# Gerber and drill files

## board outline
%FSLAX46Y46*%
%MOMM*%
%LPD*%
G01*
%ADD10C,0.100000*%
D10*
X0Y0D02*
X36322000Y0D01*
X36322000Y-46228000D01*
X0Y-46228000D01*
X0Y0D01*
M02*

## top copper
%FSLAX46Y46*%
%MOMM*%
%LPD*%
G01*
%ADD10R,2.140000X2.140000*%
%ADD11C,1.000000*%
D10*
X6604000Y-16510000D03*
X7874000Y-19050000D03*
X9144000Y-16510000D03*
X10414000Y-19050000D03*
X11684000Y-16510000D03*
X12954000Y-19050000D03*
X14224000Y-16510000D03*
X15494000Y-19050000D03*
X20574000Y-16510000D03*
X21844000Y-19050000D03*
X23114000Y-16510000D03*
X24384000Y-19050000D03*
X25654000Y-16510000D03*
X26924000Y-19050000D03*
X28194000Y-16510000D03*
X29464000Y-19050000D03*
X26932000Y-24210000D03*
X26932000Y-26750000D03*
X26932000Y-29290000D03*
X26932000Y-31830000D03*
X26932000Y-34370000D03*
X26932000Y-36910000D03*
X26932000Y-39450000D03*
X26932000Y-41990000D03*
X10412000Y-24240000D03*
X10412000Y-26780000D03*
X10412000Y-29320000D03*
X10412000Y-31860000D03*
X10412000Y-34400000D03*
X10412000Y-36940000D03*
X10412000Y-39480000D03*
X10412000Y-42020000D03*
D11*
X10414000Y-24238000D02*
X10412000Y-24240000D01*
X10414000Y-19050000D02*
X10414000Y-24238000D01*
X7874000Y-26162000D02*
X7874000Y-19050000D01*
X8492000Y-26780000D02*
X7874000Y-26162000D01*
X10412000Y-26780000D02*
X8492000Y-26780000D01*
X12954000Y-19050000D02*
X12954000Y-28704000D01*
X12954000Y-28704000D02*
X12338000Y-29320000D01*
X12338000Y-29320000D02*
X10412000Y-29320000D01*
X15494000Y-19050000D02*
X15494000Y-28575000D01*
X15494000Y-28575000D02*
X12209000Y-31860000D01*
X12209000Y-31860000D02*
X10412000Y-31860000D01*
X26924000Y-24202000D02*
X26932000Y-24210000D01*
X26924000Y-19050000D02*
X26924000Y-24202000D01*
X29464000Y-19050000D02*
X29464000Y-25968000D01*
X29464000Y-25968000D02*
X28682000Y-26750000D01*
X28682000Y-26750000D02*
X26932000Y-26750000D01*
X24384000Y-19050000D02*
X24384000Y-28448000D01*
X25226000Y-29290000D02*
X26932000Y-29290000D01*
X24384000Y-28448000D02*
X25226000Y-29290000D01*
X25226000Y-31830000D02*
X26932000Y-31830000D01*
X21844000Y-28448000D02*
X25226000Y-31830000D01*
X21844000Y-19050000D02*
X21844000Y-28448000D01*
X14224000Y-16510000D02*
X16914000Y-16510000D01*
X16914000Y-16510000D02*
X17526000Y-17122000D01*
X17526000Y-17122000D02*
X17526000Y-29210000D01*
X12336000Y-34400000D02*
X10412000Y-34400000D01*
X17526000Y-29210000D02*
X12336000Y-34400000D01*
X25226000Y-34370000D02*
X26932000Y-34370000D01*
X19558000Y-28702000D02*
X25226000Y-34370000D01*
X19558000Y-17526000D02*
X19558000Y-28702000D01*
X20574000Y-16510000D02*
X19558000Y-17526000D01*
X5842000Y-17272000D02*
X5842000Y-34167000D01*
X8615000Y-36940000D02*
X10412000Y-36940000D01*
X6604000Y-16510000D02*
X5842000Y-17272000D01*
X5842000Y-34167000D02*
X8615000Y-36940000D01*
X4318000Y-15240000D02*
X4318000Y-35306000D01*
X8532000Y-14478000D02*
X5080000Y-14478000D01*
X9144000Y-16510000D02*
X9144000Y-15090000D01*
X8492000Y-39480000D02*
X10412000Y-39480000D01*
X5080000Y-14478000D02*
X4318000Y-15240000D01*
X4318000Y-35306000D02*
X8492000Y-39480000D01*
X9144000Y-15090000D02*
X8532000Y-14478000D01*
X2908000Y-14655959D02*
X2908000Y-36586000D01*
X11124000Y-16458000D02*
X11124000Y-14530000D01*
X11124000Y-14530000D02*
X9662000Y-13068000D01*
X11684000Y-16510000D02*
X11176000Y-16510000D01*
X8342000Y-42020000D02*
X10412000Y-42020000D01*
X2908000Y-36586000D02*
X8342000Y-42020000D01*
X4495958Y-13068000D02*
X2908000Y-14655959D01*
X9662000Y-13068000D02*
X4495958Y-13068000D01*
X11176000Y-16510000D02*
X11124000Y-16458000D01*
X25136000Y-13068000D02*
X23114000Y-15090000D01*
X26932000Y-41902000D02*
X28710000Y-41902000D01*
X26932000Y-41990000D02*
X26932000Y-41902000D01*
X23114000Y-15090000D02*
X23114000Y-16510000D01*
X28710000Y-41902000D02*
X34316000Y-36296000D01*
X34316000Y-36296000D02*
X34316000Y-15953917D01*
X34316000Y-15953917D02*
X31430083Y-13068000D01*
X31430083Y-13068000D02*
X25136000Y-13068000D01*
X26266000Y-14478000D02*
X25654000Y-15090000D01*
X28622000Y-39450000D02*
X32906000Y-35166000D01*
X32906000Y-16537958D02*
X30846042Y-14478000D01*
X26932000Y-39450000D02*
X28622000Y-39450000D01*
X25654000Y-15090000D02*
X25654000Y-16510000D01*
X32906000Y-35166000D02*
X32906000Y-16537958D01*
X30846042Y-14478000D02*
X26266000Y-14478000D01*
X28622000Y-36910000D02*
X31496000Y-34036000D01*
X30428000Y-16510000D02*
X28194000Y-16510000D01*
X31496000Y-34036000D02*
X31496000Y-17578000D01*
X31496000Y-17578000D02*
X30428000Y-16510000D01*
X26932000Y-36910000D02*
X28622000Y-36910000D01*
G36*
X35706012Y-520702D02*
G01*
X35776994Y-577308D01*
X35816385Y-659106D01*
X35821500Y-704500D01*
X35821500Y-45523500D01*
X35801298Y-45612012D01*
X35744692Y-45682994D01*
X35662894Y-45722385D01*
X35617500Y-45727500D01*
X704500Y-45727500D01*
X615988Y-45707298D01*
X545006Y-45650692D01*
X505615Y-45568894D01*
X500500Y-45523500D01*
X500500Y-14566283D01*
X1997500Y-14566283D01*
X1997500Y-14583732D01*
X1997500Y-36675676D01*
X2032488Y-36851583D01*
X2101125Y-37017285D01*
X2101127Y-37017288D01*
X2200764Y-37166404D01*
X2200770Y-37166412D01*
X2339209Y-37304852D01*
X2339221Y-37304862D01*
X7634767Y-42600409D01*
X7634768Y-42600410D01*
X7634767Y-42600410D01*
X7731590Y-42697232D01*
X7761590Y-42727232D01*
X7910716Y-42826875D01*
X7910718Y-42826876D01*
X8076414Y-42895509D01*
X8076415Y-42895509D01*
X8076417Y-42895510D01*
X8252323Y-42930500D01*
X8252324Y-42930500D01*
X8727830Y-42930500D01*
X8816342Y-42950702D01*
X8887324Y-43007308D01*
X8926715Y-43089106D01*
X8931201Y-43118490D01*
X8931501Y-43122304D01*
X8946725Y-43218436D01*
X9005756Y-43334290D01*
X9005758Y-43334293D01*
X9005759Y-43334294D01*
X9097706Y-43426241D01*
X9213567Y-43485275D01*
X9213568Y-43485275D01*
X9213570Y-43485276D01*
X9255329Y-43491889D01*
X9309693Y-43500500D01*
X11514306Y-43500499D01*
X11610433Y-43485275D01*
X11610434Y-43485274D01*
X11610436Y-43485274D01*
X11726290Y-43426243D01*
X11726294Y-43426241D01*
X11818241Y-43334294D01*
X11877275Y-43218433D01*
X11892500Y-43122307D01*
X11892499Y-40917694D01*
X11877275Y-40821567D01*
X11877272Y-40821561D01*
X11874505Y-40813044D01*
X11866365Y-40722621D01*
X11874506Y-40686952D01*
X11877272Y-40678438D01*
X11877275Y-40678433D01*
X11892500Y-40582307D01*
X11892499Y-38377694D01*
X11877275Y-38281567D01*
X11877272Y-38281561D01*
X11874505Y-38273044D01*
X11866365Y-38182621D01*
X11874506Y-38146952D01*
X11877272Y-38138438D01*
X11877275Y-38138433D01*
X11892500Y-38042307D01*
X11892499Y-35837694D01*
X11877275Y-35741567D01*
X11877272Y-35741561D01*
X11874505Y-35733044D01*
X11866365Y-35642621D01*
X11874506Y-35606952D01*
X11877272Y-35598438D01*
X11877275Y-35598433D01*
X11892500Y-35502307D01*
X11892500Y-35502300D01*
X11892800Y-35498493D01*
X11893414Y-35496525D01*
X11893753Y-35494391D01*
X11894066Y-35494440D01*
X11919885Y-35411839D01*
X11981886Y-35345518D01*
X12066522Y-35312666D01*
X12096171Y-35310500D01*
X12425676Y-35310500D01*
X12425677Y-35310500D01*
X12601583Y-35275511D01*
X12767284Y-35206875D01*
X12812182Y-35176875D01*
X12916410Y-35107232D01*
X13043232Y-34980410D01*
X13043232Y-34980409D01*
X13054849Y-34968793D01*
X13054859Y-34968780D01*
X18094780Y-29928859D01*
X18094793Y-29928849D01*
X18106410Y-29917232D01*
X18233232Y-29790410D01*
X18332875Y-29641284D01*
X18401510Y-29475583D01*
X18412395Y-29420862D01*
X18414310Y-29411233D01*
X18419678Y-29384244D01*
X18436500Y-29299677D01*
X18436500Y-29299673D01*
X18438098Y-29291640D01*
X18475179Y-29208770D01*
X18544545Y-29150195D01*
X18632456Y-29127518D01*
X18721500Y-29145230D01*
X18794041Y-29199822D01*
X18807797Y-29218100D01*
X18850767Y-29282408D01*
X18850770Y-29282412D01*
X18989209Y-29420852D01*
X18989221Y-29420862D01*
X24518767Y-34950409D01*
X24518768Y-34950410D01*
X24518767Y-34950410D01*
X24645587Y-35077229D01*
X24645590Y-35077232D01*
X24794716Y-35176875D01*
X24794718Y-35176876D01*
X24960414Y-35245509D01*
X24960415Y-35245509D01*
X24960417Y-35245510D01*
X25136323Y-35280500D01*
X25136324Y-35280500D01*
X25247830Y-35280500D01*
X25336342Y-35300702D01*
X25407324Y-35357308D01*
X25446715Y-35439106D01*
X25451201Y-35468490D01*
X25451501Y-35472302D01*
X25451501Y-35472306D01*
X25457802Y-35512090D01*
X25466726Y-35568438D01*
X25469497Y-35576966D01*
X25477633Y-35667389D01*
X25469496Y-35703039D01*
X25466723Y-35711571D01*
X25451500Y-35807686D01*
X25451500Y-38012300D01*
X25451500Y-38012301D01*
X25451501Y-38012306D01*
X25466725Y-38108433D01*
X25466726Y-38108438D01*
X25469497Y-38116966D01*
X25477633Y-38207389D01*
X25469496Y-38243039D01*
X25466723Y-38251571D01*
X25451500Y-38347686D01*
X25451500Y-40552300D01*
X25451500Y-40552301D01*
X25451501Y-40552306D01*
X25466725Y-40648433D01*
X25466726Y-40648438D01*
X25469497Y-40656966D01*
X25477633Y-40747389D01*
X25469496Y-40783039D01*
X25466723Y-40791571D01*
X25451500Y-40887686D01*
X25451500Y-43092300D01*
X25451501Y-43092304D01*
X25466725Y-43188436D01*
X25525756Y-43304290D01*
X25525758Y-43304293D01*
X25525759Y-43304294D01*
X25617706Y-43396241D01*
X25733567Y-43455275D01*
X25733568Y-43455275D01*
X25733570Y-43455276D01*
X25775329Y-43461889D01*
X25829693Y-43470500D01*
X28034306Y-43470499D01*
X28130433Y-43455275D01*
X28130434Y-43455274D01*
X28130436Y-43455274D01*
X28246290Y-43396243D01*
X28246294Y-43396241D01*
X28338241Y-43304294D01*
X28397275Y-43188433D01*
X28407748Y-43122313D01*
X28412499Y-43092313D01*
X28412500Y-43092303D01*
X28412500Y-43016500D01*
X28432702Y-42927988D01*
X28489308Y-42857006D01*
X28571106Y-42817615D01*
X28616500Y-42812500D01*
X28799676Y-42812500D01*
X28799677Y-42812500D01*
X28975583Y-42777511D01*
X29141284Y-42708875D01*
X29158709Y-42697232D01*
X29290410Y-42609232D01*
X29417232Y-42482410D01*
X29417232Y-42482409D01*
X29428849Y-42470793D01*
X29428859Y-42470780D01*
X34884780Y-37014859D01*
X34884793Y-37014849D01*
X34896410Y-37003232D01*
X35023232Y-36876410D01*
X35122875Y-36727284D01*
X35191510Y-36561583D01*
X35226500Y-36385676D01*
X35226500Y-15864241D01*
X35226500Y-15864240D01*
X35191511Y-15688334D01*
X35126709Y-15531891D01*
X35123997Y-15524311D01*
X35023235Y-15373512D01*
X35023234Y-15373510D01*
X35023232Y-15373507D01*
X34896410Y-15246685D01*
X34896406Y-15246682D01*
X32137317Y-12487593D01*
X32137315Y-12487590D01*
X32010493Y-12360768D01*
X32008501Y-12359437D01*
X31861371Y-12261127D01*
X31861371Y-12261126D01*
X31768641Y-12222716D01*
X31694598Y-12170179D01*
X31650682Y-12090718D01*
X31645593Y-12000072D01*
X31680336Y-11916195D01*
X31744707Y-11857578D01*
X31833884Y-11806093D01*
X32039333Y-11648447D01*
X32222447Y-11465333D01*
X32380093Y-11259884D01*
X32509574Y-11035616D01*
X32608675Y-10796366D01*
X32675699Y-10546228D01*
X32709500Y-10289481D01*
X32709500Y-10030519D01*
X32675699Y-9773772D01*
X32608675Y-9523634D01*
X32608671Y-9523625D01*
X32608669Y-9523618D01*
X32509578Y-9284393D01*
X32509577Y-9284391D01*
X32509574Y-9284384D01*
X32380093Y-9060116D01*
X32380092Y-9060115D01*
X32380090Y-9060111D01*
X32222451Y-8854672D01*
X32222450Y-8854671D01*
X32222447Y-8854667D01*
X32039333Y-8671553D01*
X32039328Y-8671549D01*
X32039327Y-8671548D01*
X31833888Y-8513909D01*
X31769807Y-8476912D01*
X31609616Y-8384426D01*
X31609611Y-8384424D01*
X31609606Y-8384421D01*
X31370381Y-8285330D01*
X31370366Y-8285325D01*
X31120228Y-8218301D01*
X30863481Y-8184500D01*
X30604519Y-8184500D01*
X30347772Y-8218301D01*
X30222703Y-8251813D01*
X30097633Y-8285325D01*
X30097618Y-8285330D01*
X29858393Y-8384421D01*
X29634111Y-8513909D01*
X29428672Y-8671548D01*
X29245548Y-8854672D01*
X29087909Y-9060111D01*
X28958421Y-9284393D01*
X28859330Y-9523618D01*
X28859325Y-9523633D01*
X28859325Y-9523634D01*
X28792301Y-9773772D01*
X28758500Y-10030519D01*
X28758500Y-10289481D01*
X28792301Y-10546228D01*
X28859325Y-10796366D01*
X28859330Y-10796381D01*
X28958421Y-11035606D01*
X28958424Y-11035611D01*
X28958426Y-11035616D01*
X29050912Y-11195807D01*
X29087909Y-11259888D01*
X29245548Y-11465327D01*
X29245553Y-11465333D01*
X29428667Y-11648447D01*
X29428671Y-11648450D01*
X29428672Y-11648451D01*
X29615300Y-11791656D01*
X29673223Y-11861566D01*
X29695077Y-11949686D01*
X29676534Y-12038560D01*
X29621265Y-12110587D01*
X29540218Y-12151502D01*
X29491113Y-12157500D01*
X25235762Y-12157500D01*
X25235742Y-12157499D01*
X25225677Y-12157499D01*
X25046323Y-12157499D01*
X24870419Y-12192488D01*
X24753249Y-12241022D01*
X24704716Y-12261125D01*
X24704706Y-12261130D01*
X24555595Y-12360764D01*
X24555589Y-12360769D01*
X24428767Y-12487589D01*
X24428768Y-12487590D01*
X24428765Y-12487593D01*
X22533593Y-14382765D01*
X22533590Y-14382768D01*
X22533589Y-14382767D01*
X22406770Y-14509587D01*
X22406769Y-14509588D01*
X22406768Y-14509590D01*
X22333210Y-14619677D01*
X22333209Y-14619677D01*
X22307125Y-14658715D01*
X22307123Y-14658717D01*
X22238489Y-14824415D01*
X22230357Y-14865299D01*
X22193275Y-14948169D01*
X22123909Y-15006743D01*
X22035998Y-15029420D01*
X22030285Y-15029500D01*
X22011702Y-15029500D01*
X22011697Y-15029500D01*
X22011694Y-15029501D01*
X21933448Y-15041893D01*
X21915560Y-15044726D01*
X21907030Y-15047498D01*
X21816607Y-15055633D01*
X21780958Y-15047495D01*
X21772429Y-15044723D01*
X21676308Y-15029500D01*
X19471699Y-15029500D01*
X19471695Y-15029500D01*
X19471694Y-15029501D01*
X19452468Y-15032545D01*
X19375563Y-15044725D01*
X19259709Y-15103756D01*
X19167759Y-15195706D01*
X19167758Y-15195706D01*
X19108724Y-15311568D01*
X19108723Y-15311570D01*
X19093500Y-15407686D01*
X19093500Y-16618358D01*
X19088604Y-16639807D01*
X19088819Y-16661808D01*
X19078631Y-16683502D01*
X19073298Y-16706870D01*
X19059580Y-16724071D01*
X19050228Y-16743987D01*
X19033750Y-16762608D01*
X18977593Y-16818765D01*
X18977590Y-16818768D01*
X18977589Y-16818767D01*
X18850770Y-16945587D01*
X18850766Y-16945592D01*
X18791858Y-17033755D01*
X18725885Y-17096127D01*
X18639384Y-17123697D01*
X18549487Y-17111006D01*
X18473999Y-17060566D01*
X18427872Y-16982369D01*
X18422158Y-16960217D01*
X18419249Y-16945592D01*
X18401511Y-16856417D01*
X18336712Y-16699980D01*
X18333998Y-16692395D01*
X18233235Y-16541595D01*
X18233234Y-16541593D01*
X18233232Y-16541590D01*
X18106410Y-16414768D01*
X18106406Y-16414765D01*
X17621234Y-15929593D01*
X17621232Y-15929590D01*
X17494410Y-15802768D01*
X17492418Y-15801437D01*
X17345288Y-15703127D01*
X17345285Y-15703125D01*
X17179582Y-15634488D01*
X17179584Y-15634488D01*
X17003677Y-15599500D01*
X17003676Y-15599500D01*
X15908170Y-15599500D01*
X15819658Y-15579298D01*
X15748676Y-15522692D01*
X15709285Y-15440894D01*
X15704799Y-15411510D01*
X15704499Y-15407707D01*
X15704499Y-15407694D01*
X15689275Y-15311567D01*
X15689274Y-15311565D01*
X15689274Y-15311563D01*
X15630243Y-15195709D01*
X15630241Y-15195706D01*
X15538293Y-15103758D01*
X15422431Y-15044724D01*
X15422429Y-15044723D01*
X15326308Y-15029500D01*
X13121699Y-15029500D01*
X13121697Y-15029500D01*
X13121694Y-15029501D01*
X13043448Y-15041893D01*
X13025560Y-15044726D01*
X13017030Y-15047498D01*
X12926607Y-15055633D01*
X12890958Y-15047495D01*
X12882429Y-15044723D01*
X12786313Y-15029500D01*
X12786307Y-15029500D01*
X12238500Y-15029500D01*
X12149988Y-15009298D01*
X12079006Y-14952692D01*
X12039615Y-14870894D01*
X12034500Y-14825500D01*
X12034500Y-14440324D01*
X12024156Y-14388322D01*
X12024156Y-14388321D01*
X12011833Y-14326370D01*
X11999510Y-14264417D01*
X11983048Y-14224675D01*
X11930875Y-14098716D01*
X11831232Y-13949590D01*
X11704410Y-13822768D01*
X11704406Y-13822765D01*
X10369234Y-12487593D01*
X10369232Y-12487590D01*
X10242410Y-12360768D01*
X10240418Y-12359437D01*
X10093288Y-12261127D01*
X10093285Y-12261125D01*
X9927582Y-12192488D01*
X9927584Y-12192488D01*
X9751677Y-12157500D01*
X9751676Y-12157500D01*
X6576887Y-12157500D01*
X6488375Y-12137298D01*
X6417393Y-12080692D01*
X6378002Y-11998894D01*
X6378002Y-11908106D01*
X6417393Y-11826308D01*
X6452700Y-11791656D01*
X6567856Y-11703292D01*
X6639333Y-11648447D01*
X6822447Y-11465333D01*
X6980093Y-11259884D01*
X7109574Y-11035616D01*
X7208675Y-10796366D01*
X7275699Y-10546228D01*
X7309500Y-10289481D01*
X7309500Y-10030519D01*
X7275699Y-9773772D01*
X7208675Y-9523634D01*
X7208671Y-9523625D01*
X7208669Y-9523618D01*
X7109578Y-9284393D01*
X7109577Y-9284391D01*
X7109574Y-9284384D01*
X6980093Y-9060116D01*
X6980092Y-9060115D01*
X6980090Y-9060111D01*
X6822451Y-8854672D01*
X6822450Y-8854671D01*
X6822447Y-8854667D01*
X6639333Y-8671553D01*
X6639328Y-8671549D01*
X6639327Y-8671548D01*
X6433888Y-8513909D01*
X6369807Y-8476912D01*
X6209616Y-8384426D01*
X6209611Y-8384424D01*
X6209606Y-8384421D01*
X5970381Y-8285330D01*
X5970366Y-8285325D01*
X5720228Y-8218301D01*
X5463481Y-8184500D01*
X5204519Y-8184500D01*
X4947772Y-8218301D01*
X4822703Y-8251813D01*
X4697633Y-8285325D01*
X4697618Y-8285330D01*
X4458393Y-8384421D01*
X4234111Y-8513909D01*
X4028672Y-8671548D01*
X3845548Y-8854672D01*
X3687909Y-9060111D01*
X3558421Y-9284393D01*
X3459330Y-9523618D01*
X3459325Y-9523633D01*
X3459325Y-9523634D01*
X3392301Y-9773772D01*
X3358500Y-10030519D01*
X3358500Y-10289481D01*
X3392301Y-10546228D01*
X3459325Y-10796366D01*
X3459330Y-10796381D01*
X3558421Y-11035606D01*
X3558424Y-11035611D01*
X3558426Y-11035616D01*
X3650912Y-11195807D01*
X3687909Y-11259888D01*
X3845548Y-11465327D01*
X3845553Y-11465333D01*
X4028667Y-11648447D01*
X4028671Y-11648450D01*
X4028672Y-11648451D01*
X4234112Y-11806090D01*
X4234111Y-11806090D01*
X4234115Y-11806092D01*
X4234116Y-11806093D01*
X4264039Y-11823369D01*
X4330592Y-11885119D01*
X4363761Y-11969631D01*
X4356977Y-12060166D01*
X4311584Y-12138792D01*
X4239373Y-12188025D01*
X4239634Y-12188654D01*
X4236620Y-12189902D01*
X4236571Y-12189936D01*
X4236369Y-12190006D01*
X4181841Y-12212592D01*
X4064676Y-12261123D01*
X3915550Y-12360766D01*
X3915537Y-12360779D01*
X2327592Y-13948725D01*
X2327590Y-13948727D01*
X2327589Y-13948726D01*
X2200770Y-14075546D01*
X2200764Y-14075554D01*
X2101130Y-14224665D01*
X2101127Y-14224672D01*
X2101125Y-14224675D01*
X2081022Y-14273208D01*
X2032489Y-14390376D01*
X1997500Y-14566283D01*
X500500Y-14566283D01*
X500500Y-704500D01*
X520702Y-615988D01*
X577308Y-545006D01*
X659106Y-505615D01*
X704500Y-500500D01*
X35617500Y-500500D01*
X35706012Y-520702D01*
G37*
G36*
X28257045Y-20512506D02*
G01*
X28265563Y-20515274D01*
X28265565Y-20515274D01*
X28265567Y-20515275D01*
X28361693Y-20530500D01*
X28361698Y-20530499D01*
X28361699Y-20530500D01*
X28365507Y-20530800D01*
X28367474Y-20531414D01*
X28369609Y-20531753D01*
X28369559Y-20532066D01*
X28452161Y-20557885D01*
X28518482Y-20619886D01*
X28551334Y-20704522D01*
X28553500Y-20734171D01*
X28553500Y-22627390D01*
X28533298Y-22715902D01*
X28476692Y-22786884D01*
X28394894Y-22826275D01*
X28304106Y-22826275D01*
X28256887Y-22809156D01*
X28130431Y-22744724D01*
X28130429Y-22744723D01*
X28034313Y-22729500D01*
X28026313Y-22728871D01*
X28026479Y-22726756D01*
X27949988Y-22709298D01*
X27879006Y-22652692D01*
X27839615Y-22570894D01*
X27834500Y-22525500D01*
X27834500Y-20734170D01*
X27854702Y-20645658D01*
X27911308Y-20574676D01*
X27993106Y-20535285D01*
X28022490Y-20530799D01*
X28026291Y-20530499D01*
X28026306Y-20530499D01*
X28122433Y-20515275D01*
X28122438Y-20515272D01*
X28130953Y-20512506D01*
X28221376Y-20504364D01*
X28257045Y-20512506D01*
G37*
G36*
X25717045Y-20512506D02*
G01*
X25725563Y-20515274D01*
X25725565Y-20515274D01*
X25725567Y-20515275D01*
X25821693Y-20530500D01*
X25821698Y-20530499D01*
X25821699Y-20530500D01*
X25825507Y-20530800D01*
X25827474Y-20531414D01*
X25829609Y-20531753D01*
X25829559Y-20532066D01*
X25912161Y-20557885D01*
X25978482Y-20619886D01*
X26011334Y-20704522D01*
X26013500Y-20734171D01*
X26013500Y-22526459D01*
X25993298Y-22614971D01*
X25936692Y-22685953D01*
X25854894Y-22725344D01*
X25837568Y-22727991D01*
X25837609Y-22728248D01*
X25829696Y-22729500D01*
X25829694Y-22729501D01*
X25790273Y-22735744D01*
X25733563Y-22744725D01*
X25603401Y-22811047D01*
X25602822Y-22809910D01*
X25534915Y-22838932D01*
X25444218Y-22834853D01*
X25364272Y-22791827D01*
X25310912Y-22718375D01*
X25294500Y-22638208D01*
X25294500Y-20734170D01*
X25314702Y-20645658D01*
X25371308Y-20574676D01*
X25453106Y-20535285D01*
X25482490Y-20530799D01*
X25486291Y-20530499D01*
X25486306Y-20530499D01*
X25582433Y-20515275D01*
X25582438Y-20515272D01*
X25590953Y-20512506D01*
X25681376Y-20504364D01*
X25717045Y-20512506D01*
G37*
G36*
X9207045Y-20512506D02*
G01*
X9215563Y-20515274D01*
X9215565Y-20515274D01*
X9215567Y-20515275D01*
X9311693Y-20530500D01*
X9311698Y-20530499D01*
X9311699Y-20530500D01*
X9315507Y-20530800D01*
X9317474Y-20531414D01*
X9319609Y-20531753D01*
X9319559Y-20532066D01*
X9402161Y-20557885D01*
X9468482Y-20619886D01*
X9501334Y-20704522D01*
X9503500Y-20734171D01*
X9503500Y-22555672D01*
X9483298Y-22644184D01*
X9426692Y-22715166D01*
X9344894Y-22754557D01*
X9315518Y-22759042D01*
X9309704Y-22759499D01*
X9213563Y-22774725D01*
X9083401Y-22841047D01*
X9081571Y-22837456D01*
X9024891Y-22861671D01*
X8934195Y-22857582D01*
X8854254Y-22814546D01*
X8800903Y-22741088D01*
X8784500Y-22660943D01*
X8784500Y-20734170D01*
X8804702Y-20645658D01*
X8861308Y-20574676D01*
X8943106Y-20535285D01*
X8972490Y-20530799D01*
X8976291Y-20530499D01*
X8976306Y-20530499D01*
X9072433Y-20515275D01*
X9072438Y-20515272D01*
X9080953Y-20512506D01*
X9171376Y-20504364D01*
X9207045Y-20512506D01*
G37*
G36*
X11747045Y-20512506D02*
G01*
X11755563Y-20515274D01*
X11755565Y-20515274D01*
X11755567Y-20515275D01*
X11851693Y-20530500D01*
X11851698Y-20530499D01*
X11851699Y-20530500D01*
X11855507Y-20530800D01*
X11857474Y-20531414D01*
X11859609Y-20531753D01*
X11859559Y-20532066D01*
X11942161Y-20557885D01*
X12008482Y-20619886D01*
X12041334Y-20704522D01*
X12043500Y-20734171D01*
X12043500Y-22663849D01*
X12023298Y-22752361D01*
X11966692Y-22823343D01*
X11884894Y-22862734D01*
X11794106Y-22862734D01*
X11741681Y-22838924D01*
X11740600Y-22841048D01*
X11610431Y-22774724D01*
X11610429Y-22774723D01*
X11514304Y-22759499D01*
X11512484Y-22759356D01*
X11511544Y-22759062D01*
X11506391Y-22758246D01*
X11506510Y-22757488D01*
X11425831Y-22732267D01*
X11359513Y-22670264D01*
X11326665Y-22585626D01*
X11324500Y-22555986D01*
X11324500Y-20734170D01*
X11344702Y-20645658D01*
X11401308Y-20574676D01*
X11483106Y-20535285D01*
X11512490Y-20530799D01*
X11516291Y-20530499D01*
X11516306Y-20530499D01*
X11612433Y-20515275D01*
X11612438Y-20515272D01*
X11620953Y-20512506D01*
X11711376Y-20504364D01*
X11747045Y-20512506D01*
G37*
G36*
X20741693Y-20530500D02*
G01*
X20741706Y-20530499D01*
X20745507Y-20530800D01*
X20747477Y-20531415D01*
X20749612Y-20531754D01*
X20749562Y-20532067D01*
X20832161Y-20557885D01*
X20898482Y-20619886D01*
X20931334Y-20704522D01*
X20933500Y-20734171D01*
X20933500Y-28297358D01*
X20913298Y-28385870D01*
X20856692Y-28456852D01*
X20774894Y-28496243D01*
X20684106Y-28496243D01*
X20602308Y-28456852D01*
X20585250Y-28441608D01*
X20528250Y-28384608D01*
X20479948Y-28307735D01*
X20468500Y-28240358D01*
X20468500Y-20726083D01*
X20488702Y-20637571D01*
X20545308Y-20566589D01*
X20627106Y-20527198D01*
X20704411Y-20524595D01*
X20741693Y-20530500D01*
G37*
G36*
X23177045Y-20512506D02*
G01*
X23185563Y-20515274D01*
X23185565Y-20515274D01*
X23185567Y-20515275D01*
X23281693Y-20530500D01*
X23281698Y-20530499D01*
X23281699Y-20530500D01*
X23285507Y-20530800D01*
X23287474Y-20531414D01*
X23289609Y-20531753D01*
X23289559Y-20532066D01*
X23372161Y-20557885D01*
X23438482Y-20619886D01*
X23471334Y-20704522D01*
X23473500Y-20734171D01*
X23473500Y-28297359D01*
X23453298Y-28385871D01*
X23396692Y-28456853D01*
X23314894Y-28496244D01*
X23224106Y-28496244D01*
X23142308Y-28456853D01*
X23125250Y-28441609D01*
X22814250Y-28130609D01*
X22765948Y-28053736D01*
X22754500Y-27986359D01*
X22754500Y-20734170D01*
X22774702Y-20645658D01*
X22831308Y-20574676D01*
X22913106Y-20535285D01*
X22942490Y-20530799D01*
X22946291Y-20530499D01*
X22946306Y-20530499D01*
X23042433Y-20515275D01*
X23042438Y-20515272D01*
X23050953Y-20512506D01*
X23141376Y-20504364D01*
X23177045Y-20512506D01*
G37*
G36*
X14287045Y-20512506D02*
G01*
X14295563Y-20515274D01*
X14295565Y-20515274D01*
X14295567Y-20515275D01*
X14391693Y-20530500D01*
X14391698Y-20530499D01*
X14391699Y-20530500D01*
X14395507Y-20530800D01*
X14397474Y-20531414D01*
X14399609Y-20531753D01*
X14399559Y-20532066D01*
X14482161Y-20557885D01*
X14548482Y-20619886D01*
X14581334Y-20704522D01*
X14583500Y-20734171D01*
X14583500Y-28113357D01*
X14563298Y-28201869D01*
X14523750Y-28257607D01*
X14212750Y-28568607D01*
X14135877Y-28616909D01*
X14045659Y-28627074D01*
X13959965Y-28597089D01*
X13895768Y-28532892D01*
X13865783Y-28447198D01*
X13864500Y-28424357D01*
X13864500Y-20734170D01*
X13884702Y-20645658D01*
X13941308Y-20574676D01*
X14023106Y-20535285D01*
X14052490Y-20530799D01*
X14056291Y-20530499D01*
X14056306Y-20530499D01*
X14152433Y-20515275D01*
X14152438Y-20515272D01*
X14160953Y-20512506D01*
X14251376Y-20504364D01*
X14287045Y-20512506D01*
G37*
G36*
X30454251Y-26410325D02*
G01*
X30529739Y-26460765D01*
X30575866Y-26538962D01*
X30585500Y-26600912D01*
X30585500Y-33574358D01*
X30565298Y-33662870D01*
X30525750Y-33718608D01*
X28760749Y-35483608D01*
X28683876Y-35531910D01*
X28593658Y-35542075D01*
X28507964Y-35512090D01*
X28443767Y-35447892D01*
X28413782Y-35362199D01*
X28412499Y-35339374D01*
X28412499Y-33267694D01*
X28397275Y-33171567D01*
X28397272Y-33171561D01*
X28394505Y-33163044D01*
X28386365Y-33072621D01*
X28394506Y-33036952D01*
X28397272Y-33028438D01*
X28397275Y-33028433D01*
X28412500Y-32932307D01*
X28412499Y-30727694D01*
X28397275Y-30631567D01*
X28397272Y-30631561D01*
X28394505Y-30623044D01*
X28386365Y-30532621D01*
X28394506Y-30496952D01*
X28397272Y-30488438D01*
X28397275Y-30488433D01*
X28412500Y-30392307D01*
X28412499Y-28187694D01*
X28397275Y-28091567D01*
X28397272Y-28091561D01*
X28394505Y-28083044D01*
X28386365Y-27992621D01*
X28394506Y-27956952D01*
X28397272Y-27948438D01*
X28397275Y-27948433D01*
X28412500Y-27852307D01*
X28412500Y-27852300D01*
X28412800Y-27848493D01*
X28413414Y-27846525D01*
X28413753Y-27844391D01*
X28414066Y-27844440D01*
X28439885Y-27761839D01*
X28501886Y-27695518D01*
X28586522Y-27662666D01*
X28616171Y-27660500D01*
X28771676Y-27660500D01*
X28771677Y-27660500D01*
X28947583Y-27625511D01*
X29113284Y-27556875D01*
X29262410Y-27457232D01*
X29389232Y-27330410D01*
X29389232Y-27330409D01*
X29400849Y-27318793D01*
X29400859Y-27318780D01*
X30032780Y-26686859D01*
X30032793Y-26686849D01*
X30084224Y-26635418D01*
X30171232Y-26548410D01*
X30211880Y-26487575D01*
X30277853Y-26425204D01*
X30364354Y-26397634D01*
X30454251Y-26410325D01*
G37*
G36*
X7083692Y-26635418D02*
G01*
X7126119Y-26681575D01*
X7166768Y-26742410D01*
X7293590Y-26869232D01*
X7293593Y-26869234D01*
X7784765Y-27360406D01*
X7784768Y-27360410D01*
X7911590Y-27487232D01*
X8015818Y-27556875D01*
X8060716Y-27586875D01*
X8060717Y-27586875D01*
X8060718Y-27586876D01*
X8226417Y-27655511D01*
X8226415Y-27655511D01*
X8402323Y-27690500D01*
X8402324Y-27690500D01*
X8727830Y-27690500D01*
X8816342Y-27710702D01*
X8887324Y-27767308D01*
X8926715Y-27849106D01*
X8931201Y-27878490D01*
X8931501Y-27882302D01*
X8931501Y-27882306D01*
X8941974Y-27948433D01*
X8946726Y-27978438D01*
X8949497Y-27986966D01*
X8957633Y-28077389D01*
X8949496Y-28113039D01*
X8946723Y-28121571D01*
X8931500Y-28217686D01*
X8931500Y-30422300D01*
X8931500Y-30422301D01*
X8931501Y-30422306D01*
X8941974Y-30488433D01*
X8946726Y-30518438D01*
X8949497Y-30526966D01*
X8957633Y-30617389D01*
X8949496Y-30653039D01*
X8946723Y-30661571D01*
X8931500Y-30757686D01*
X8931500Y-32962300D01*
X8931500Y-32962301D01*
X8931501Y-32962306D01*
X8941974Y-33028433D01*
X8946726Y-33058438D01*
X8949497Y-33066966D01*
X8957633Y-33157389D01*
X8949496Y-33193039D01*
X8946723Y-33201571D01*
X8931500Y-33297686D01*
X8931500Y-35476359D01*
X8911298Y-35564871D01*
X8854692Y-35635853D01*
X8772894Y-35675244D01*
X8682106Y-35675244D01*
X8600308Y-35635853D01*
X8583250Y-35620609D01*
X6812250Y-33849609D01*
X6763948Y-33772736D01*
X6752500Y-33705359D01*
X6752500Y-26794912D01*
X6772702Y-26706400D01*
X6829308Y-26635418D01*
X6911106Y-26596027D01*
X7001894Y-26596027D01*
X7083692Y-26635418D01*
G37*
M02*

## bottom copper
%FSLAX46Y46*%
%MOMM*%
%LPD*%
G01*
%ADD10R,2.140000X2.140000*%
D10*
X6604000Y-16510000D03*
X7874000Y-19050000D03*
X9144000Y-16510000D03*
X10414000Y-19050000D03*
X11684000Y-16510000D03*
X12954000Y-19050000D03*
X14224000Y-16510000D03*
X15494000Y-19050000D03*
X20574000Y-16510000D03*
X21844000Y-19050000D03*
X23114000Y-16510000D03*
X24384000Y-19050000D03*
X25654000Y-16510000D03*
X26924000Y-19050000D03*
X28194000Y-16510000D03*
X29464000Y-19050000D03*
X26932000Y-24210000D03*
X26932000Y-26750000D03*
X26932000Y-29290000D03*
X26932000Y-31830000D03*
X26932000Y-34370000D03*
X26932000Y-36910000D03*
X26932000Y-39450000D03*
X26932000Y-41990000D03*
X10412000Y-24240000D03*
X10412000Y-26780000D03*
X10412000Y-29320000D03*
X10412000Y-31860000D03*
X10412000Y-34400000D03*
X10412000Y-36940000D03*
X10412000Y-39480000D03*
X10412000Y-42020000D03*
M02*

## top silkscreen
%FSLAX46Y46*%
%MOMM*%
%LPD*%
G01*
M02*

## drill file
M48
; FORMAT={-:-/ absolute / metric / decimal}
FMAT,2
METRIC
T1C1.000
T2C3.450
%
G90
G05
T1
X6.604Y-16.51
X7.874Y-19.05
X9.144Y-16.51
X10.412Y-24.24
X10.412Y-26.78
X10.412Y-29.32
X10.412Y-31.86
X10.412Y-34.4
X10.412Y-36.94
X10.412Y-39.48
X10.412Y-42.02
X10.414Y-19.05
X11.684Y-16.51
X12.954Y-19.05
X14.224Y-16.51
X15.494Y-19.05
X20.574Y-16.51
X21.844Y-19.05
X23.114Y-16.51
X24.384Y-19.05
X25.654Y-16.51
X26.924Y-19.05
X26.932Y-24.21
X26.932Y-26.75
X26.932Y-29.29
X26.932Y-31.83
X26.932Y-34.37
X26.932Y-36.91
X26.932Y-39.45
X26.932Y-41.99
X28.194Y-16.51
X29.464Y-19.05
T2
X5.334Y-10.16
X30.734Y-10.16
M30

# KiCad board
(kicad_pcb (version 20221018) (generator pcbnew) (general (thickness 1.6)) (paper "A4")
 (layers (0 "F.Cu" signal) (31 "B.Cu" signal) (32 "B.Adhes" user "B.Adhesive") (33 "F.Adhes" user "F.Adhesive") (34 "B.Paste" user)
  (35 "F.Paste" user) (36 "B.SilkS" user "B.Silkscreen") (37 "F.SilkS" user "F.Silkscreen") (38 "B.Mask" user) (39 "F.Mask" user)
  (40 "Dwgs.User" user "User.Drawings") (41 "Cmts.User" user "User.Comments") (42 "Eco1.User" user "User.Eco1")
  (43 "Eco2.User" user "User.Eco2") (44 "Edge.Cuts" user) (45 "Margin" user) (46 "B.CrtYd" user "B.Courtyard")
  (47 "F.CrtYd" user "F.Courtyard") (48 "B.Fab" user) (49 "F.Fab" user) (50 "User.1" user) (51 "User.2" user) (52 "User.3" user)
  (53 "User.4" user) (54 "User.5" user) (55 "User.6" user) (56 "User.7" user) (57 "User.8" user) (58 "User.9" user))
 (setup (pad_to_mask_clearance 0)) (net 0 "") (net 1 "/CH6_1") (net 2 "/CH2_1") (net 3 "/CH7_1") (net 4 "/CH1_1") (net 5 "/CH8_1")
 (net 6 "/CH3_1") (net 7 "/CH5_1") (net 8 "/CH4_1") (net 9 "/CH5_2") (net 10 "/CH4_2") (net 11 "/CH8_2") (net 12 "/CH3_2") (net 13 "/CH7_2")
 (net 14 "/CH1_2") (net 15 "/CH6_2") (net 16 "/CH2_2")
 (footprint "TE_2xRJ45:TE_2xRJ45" (layer "B.Cu") (at 18.034 10.435)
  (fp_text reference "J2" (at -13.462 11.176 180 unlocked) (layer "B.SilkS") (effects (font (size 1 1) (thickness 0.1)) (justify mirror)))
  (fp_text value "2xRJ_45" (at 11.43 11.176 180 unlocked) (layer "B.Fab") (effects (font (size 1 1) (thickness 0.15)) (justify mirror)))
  (pad "" np_thru_hole circle (at -12.7 -0.275) (size 3.25 3.25) (drill 3.45) (layers "F&B.Cu" "*.Mask"))
  (pad "" np_thru_hole circle (at 12.7 -0.275) (size 3.45 3.45) (drill 3.45) (layers "F&B.Cu" "*.Mask"))
  (pad "1_1" thru_hole rect (at -11.43 6.075) (size 2.14 2.14) (drill 1) (layers "*.Cu" "*.Mask") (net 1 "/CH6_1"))
  (pad "1_2" thru_hole rect (at -10.16 8.615) (size 2.14 2.14) (drill 1) (layers "*.Cu" "*.Mask") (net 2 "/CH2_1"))
  (pad "1_3" thru_hole rect (at -8.89 6.075) (size 2.14 2.14) (drill 1) (layers "*.Cu" "*.Mask") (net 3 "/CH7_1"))
  (pad "1_4" thru_hole rect (at -7.62 8.615) (size 2.14 2.14) (drill 1) (layers "*.Cu" "*.Mask") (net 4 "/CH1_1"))
  (pad "1_5" thru_hole rect (at -6.35 6.075) (size 2.14 2.14) (drill 1) (layers "*.Cu" "*.Mask") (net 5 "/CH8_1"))
  (pad "1_6" thru_hole rect (at -5.08 8.615) (size 2.14 2.14) (drill 1) (layers "*.Cu" "*.Mask") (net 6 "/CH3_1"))
  (pad "1_7" thru_hole rect (at -3.81 6.075) (size 2.14 2.14) (drill 1) (layers "*.Cu" "*.Mask") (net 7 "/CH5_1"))
  (pad "1_8" thru_hole rect (at -2.54 8.615) (size 2.14 2.14) (drill 1) (layers "*.Cu" "*.Mask") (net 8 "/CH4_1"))
  (pad "2_1" thru_hole rect (at 2.54 6.075) (size 2.14 2.14) (drill 1) (layers "*.Cu" "*.Mask") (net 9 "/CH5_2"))
  (pad "2_2" thru_hole rect (at 3.81 8.615) (size 2.14 2.14) (drill 1) (layers "*.Cu" "*.Mask") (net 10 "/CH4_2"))
  (pad "2_3" thru_hole rect (at 5.08 6.075) (size 2.14 2.14) (drill 1) (layers "*.Cu" "*.Mask") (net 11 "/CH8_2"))
  (pad "2_4" thru_hole rect (at 6.35 8.615) (size 2.14 2.14) (drill 1) (layers "*.Cu" "*.Mask") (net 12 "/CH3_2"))
  (pad "2_5" thru_hole rect (at 7.62 6.075) (size 2.14 2.14) (drill 1) (layers "*.Cu" "*.Mask") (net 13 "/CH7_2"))
  (pad "2_6" thru_hole rect (at 8.89 8.615) (size 2.14 2.14) (drill 1) (layers "*.Cu" "*.Mask") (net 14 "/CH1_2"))
  (pad "2_7" thru_hole rect (at 10.16 6.075) (size 2.14 2.14) (drill 1) (layers "*.Cu" "*.Mask") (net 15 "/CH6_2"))
  (pad "2_8" thru_hole rect (at 11.43 8.615) (size 2.14 2.14) (drill 1) (layers "*.Cu" "*.Mask") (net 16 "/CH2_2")))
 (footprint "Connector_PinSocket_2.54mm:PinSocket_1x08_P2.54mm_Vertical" (layer "B.Cu") (at 26.932 24.21 180)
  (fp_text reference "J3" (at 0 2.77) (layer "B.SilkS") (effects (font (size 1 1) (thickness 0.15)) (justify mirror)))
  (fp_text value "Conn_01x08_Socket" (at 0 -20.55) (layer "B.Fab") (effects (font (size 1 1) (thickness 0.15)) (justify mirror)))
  (pad "1" thru_hole rect (at 0 0 180) (size 2.14 2.14) (drill 1) (layers "*.Cu" "*.Mask") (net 14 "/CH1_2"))
  (pad "2" thru_hole rect (at 0 -2.54 180) (size 2.14 2.14) (drill 1) (layers "*.Cu" "*.Mask") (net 16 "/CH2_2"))
  (pad "3" thru_hole rect (at 0 -5.08 180) (size 2.14 2.14) (drill 1) (layers "*.Cu" "*.Mask") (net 12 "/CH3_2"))
  (pad "4" thru_hole rect (at 0 -7.62 180) (size 2.14 2.14) (drill 1) (layers "*.Cu" "*.Mask") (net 10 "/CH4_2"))
  (pad "5" thru_hole rect (at 0 -10.16 180) (size 2.14 2.14) (drill 1) (layers "*.Cu" "*.Mask") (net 9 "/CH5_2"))
  (pad "6" thru_hole rect (at 0 -12.7 180) (size 2.14 2.14) (drill 1) (layers "*.Cu" "*.Mask") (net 15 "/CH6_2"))
  (pad "7" thru_hole rect (at 0 -15.24 180) (size 2.14 2.14) (drill 1) (layers "*.Cu" "*.Mask") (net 13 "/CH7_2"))
  (pad "8" thru_hole rect (at 0 -17.78 180) (size 2.14 2.14) (drill 1) (layers "*.Cu" "*.Mask") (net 11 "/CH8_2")))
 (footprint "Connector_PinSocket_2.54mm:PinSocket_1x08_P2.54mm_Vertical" (layer "B.Cu") (at 10.412 24.24 180)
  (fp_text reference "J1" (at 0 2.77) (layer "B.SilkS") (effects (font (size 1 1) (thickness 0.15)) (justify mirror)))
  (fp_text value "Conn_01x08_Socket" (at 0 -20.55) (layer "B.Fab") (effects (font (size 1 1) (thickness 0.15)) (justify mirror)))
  (pad "1" thru_hole rect (at 0 0 180) (size 2.14 2.14) (drill 1) (layers "*.Cu" "*.Mask") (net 4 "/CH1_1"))
  (pad "2" thru_hole rect (at 0 -2.54 180) (size 2.14 2.14) (drill 1) (layers "*.Cu" "*.Mask") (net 2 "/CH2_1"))
  (pad "3" thru_hole rect (at 0 -5.08 180) (size 2.14 2.14) (drill 1) (layers "*.Cu" "*.Mask") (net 6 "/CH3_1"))
  (pad "4" thru_hole rect (at 0 -7.62 180) (size 2.14 2.14) (drill 1) (layers "*.Cu" "*.Mask") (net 8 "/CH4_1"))
  (pad "5" thru_hole rect (at 0 -10.16 180) (size 2.14 2.14) (drill 1) (layers "*.Cu" "*.Mask") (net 7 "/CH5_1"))
  (pad "6" thru_hole rect (at 0 -12.7 180) (size 2.14 2.14) (drill 1) (layers "*.Cu" "*.Mask") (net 1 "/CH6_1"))
  (pad "7" thru_hole rect (at 0 -15.24 180) (size 2.14 2.14) (drill 1) (layers "*.Cu" "*.Mask") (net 3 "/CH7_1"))
  (pad "8" thru_hole rect (at 0 -17.78 180) (size 2.14 2.14) (drill 1) (layers "*.Cu" "*.Mask") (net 5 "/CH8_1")))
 (gr_rect (start 0 0) (end 36.322 46.228) (stroke (width 0.1) (type default)) (fill none) (layer "Edge.Cuts"))
 (segment (start 10.414 24.238) (end 10.412 24.24) (width 1) (layer "F.Cu") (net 4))
 (segment (start 10.414 19.05) (end 10.414 24.238) (width 1) (layer "F.Cu") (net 4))
 (segment (start 7.874 26.162) (end 7.874 19.05) (width 1) (layer "F.Cu") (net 2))
 (segment (start 8.492 26.78) (end 7.874 26.162) (width 1) (layer "F.Cu") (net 2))
 (segment (start 10.412 26.78) (end 8.492 26.78) (width 1) (layer "F.Cu") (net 2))
 (segment (start 12.954 19.05) (end 12.954 28.704) (width 1) (layer "F.Cu") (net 6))
 (segment (start 12.954 28.704) (end 12.338 29.32) (width 1) (layer "F.Cu") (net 6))
 (segment (start 12.338 29.32) (end 10.412 29.32) (width 1) (layer "F.Cu") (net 6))
 (segment (start 15.494 19.05) (end 15.494 28.575) (width 1) (layer "F.Cu") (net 8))
 (segment (start 15.494 28.575) (end 12.209 31.86) (width 1) (layer "F.Cu") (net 8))
 (segment (start 12.209 31.86) (end 10.412 31.86) (width 1) (layer "F.Cu") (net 8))
 (segment (start 26.924 24.202) (end 26.932 24.21) (width 1) (layer "F.Cu") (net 14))
 (segment (start 26.924 19.05) (end 26.924 24.202) (width 1) (layer "F.Cu") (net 14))
 (segment (start 29.464 19.05) (end 29.464 25.968) (width 1) (layer "F.Cu") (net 16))
 (segment (start 29.464 25.968) (end 28.682 26.75) (width 1) (layer "F.Cu") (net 16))
 (segment (start 28.682 26.75) (end 26.932 26.75) (width 1) (layer "F.Cu") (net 16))
 (segment (start 24.384 19.05) (end 24.384 28.448) (width 1) (layer "F.Cu") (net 12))
 (segment (start 25.226 29.29) (end 26.932 29.29) (width 1) (layer "F.Cu") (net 12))
 (segment (start 24.384 28.448) (end 25.226 29.29) (width 1) (layer "F.Cu") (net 12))
 (segment (start 25.226 31.83) (end 26.932 31.83) (width 1) (layer "F.Cu") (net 10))
 (segment (start 21.844 28.448) (end 25.226 31.83) (width 1) (layer "F.Cu") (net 10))
 (segment (start 21.844 19.05) (end 21.844 28.448) (width 1) (layer "F.Cu") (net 10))
 (segment (start 14.224 16.51) (end 16.914 16.51) (width 1) (layer "F.Cu") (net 7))
 (segment (start 16.914 16.51) (end 17.526 17.122) (width 1) (layer "F.Cu") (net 7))
 (segment (start 17.526 17.122) (end 17.526 29.21) (width 1) (layer "F.Cu") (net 7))
 (segment (start 12.336 34.4) (end 10.412 34.4) (width 1) (layer "F.Cu") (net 7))
 (segment (start 17.526 29.21) (end 12.336 34.4) (width 1) (layer "F.Cu") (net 7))
 (segment (start 25.226 34.37) (end 26.932 34.37) (width 1) (layer "F.Cu") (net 9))
 (segment (start 19.558 28.702) (end 25.226 34.37) (width 1) (layer "F.Cu") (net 9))
 (segment (start 19.558 17.526) (end 19.558 28.702) (width 1) (layer "F.Cu") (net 9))
 (segment (start 20.574 16.51) (end 19.558 17.526) (width 1) (layer "F.Cu") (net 9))
 (segment (start 5.842 17.272) (end 5.842 34.167) (width 1) (layer "F.Cu") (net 1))
 (segment (start 8.615 36.94) (end 10.412 36.94) (width 1) (layer "F.Cu") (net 1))
 (segment (start 6.604 16.51) (end 5.842 17.272) (width 1) (layer "F.Cu") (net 1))
 (segment (start 5.842 34.167) (end 8.615 36.94) (width 1) (layer "F.Cu") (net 1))
 (segment (start 4.318 15.24) (end 4.318 35.306) (width 1) (layer "F.Cu") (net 3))
 (segment (start 8.532 14.478) (end 5.08 14.478) (width 1) (layer "F.Cu") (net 3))
 (segment (start 9.144 16.51) (end 9.144 15.09) (width 1) (layer "F.Cu") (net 3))
 (segment (start 8.492 39.48) (end 10.412 39.48) (width 1) (layer "F.Cu") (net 3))
 (segment (start 5.08 14.478) (end 4.318 15.24) (width 1) (layer "F.Cu") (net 3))
 (segment (start 4.318 35.306) (end 8.492 39.48) (width 1) (layer "F.Cu") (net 3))
 (segment (start 9.144 15.09) (end 8.532 14.478) (width 1) (layer "F.Cu") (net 3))
 (segment (start 2.908 14.655959) (end 2.908 36.586) (width 1) (layer "F.Cu") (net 5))
 (segment (start 11.124 16.458) (end 11.124 14.53) (width 1) (layer "F.Cu") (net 5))
 (segment (start 11.124 14.53) (end 9.662 13.068) (width 1) (layer "F.Cu") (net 5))
 (segment (start 11.684 16.51) (end 11.176 16.51) (width 1) (layer "F.Cu") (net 5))
 (segment (start 8.342 42.02) (end 10.412 42.02) (width 1) (layer "F.Cu") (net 5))
 (segment (start 2.908 36.586) (end 8.342 42.02) (width 1) (layer "F.Cu") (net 5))
 (segment (start 4.495958 13.068) (end 2.908 14.655959) (width 1) (layer "F.Cu") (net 5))
 (segment (start 9.662 13.068) (end 4.495958 13.068) (width 1) (layer "F.Cu") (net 5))
 (segment (start 11.176 16.51) (end 11.124 16.458) (width 1) (layer "F.Cu") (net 5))
 (segment (start 25.136 13.068) (end 23.114 15.09) (width 1) (layer "F.Cu") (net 11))
 (segment (start 26.932 41.902) (end 28.71 41.902) (width 1) (layer "F.Cu") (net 11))
 (segment (start 26.932 41.99) (end 26.932 41.902) (width 1) (layer "F.Cu") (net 11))
 (segment (start 23.114 15.09) (end 23.114 16.51) (width 1) (layer "F.Cu") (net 11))
 (segment (start 28.71 41.902) (end 34.316 36.296) (width 1) (layer "F.Cu") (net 11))
 (segment (start 34.316 36.296) (end 34.316 15.953917) (width 1) (layer "F.Cu") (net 11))
 (segment (start 34.316 15.953917) (end 31.430083 13.068) (width 1) (layer "F.Cu") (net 11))
 (segment (start 31.430083 13.068) (end 25.136 13.068) (width 1) (layer "F.Cu") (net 11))
 (segment (start 26.266 14.478) (end 25.654 15.09) (width 1) (layer "F.Cu") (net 13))
 (segment (start 28.622 39.45) (end 32.906 35.166) (width 1) (layer "F.Cu") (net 13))
 (segment (start 32.906 16.537958) (end 30.846042 14.478) (width 1) (layer "F.Cu") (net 13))
 (segment (start 26.932 39.45) (end 28.622 39.45) (width 1) (layer "F.Cu") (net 13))
 (segment (start 25.654 15.09) (end 25.654 16.51) (width 1) (layer "F.Cu") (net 13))
 (segment (start 32.906 35.166) (end 32.906 16.537958) (width 1) (layer "F.Cu") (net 13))
 (segment (start 30.846042 14.478) (end 26.266 14.478) (width 1) (layer "F.Cu") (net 13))
 (segment (start 28.622 36.91) (end 31.496 34.036) (width 1) (layer "F.Cu") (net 15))
 (segment (start 30.428 16.51) (end 28.194 16.51) (width 1) (layer "F.Cu") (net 15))
 (segment (start 31.496 34.036) (end 31.496 17.578) (width 1) (layer "F.Cu") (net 15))
 (segment (start 31.496 17.578) (end 30.428 16.51) (width 1) (layer "F.Cu") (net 15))
 (segment (start 26.932 36.91) (end 28.622 36.91) (width 1) (layer "F.Cu") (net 15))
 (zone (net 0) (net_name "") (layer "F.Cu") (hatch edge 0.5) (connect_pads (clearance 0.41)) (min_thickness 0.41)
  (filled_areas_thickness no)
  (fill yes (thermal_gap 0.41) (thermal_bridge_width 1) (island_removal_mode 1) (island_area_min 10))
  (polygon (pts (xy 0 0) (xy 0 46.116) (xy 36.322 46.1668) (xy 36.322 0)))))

